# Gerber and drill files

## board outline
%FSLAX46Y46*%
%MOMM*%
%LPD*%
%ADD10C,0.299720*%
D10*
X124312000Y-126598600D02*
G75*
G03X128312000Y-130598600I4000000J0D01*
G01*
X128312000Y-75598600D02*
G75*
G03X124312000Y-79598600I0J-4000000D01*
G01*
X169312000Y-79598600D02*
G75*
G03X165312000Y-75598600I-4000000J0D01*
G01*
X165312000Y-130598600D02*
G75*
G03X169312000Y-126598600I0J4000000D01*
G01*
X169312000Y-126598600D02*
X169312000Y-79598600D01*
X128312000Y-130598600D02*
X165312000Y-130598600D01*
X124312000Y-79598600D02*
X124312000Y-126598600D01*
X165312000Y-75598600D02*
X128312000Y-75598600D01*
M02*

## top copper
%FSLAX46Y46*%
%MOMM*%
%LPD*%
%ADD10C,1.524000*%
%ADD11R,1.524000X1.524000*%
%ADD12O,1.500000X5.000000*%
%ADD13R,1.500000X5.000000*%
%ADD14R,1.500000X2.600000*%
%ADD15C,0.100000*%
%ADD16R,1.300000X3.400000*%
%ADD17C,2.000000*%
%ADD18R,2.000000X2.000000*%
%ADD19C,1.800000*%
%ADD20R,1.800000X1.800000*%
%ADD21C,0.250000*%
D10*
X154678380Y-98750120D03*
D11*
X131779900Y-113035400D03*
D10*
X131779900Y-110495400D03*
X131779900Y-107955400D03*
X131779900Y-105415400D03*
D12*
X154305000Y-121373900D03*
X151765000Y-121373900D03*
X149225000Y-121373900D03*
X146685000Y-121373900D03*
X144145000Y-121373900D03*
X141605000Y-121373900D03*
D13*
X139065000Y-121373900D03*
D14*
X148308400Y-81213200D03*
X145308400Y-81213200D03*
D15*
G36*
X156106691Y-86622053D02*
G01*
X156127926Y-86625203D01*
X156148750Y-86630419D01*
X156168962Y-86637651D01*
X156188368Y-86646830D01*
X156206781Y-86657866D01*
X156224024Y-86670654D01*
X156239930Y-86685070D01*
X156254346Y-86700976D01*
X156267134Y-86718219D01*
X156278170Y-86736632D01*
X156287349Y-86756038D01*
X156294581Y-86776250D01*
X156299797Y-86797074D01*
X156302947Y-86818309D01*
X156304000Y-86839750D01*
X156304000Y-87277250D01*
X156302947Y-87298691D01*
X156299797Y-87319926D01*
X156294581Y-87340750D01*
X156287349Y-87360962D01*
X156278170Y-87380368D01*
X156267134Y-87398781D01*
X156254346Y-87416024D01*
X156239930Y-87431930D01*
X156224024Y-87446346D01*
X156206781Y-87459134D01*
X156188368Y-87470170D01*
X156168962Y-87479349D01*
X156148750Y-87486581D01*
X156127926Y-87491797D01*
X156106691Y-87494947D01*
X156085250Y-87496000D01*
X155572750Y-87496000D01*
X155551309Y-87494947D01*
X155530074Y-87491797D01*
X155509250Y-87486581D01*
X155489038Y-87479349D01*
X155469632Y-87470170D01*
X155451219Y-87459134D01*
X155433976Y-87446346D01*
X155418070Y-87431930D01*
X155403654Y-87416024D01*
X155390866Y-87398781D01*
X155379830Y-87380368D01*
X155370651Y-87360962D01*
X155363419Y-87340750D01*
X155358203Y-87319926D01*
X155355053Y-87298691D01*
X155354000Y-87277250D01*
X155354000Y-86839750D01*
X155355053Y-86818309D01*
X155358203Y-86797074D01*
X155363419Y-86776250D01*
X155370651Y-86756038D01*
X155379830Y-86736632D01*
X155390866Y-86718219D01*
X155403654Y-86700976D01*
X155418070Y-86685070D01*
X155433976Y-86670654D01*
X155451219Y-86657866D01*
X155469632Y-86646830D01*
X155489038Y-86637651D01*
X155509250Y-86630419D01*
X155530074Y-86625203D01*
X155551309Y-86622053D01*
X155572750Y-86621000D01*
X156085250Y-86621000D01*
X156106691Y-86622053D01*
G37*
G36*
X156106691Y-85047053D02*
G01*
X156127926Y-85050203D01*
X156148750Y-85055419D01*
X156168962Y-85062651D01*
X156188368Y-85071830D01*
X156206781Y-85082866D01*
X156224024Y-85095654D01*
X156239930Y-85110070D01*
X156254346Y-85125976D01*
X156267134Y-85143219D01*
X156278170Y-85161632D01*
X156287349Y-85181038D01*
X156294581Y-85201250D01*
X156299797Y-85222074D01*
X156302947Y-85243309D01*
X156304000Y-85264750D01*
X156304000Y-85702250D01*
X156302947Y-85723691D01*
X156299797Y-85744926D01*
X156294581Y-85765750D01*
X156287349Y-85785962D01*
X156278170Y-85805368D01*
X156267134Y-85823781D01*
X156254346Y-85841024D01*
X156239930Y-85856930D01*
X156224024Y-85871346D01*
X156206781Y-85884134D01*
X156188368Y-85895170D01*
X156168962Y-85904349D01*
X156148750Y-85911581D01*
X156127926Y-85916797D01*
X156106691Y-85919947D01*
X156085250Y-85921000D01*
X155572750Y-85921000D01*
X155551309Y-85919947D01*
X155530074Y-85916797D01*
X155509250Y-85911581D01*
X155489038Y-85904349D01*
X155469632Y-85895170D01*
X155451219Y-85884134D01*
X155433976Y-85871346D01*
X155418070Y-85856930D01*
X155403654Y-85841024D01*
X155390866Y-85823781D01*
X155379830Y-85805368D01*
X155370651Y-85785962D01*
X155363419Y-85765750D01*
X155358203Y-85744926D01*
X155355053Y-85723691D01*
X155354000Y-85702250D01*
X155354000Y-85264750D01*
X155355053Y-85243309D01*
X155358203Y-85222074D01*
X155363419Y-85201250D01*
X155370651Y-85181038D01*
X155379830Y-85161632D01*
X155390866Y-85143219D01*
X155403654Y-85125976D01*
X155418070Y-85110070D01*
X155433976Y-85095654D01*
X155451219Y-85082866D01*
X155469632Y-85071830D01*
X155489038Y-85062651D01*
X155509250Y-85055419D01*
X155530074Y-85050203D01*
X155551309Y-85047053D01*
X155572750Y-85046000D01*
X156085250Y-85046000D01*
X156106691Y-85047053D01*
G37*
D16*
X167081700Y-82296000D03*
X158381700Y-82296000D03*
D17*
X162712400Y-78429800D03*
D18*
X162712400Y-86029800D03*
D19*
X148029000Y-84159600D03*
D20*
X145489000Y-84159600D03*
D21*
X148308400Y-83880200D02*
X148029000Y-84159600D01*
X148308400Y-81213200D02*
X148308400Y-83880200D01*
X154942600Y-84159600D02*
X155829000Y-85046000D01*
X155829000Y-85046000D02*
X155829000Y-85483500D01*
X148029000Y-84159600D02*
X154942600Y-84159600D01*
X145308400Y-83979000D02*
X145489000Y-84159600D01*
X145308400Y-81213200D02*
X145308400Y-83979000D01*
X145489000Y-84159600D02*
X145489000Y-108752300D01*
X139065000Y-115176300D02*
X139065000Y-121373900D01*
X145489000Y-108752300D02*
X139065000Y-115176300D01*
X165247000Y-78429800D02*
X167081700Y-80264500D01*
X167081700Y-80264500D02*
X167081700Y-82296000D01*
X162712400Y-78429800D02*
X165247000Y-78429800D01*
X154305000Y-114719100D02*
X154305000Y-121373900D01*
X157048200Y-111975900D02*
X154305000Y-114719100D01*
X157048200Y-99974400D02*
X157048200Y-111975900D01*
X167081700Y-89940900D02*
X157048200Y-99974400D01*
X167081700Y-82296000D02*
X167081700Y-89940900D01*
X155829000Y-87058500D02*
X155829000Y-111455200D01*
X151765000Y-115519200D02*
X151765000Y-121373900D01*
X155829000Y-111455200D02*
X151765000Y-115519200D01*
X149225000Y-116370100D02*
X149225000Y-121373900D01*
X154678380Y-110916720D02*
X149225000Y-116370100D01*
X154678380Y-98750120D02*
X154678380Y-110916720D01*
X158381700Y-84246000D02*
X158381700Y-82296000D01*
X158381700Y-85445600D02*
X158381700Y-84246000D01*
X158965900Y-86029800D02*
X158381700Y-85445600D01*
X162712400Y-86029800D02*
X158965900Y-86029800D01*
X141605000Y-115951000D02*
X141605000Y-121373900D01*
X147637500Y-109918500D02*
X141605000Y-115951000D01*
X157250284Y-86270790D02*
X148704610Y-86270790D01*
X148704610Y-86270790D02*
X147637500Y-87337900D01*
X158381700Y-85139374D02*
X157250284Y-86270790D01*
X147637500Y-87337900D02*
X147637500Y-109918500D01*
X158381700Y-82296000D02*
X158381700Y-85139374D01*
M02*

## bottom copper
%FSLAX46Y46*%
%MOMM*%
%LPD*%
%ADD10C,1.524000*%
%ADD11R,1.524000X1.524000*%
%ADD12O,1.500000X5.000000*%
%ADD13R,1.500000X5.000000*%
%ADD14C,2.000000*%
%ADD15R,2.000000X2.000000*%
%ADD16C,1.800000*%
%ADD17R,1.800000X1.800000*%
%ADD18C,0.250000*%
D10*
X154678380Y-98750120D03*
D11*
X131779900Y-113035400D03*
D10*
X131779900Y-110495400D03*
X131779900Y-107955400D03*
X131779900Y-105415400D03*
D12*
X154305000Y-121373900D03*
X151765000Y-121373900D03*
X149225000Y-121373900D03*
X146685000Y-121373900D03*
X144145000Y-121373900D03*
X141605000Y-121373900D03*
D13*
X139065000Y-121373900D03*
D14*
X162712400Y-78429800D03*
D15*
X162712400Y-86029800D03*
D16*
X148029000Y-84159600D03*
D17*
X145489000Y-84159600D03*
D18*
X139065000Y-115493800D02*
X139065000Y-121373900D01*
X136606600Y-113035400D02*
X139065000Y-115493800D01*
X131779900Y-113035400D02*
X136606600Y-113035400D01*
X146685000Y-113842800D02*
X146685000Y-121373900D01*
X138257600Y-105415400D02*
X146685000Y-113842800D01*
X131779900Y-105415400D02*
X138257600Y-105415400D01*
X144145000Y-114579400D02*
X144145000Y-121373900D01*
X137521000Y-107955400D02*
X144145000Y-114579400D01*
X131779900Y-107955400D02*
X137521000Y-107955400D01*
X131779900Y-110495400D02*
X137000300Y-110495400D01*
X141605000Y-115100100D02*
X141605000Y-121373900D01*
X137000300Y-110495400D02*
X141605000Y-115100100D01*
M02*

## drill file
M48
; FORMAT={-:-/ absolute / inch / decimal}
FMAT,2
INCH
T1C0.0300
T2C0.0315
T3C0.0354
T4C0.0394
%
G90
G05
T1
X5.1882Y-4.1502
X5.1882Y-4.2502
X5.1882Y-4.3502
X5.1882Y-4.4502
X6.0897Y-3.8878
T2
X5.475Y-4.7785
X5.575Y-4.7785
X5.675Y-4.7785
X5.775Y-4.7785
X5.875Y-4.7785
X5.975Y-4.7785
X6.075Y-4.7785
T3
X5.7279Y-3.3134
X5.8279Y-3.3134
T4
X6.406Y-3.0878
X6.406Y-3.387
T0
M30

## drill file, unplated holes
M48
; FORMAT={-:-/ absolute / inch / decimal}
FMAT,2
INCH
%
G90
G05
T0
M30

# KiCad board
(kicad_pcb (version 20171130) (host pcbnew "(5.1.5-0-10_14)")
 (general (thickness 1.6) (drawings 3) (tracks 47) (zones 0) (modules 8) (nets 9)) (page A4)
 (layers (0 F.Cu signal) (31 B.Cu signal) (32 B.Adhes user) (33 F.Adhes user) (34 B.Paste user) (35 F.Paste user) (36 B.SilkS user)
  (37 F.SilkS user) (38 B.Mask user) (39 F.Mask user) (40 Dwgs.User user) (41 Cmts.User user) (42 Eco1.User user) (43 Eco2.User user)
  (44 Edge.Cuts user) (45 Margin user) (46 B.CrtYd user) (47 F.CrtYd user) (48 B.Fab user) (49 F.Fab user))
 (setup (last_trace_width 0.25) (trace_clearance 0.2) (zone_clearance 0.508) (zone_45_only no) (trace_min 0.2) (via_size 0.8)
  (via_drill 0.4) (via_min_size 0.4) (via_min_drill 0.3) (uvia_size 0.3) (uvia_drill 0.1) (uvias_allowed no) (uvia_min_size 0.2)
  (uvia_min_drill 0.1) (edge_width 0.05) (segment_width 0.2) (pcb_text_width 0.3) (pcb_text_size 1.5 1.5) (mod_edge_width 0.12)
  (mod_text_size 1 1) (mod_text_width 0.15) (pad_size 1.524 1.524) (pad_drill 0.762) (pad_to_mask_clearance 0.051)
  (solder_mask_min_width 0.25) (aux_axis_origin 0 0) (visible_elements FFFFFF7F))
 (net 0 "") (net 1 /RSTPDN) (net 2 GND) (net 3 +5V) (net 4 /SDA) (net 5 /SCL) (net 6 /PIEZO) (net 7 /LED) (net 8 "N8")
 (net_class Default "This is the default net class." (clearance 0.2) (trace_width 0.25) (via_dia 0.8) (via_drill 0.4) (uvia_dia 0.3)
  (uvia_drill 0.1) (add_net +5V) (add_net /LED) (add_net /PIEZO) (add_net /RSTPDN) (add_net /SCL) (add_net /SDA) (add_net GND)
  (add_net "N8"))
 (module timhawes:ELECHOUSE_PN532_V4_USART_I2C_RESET (layer B.Cu) (at 151.5999 109.2454 90)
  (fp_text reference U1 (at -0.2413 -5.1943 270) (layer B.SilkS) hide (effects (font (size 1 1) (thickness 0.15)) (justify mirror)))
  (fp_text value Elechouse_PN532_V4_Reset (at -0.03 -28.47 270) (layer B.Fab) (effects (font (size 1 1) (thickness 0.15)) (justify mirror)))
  (pad 5 thru_hole circle (at 10.49528 3.07848 90) (size 1.524 1.524) (drill 0.762) (layers *.Cu *.Mask) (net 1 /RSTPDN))
  (pad 1 thru_hole rect (at -3.79 -19.82 90) (size 1.524 1.524) (drill 0.762) (layers *.Cu *.Mask) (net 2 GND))
  (pad 2 thru_hole circle (at -1.25 -19.82 90) (size 1.524 1.524) (drill 0.762) (layers *.Cu *.Mask) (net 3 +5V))
  (pad 3 thru_hole circle (at 1.29 -19.82 90) (size 1.524 1.524) (drill 0.762) (layers *.Cu *.Mask) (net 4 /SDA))
  (pad 4 thru_hole circle (at 3.83 -19.82 90) (size 1.524 1.524) (drill 0.762) (layers *.Cu *.Mask) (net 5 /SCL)))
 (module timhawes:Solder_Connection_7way (layer B.Cu) (at 146.685 121.3739)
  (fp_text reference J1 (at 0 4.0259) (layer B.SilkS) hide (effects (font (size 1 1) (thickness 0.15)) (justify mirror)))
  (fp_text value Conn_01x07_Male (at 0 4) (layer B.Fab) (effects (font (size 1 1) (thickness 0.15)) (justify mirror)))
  (pad 7 thru_hole oval (at 7.62 0) (size 1.5 5) (drill 0.8) (layers *.Cu *.Mask) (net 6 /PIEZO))
  (pad 6 thru_hole oval (at 5.08 0) (size 1.5 5) (drill 0.8) (layers *.Cu *.Mask) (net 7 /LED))
  (pad 5 thru_hole oval (at 2.54 0) (size 1.5 5) (drill 0.8) (layers *.Cu *.Mask) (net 1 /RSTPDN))
  (pad 4 thru_hole oval (at 0 0) (size 1.5 5) (drill 0.8) (layers *.Cu *.Mask) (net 5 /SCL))
  (pad 3 thru_hole oval (at -2.54 0) (size 1.5 5) (drill 0.8) (layers *.Cu *.Mask) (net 4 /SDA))
  (pad 2 thru_hole oval (at -5.08 0) (size 1.5 5) (drill 0.8) (layers *.Cu *.Mask) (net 3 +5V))
  (pad 1 thru_hole rect (at -7.62 0) (size 1.5 5) (drill 0.8) (layers *.Cu *.Mask) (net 2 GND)))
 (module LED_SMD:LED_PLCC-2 (layer F.Cu) (at 146.8084 81.2132)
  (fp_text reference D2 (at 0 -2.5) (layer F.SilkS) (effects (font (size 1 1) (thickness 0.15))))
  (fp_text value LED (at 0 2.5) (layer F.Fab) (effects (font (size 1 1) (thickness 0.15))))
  (pad 2 smd rect (at 1.5 0) (size 1.5 2.6) (layers F.Cu F.Paste F.Mask) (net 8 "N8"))
  (pad 1 smd rect (at -1.5 0) (size 1.5 2.6) (layers F.Cu F.Paste F.Mask) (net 2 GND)))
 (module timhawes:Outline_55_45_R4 (layer F.Cu) (at 146.812 103.0986 90)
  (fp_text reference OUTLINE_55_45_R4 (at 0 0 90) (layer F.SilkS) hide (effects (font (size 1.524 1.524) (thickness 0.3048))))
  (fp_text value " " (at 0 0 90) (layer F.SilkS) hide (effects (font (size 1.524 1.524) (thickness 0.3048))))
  (fp_arc (start -23.5 -18.5) (end -27.5 -18.5) (angle 90) (layer Edge.Cuts) (width 0.29972))
  (fp_arc (start 23.5 -18.5) (end 23.5 -22.5) (angle 90) (layer Edge.Cuts) (width 0.29972))
  (fp_arc (start 23.5 18.5) (end 27.5 18.5) (angle 90) (layer Edge.Cuts) (width 0.29972))
  (fp_arc (start -23.5 18.5) (end -23.5 22.5) (angle 90) (layer Edge.Cuts) (width 0.29972))
  (fp_line (start -23.5 22.5) (end 23.5 22.5) (layer Edge.Cuts) (width 0.29972))
  (fp_line (start -27.5 -18.5) (end -27.5 18.5) (layer Edge.Cuts) (width 0.29972))
  (fp_line (start 23.5 -22.5) (end -23.5 -22.5) (layer Edge.Cuts) (width 0.29972))
  (fp_line (start 27.5 18.5) (end 27.5 -18.5) (layer Edge.Cuts) (width 0.29972)))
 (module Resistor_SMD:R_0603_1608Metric (layer F.Cu) (at 155.829 86.271 270)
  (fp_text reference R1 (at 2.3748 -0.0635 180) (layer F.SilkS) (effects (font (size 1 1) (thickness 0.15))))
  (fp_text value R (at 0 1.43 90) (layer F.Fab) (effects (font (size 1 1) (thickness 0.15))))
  (pad 2 smd roundrect (at 0.7875 0 270) (size 0.875 0.95) (layers F.Cu F.Paste F.Mask) (roundrect_rratio 0.25) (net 7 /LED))
  (pad 1 smd roundrect (at -0.7875 0 270) (size 0.875 0.95) (layers F.Cu F.Paste F.Mask) (roundrect_rratio 0.25) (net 8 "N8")))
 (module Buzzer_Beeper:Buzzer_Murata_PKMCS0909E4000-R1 (layer F.Cu) (at 162.7317 82.296)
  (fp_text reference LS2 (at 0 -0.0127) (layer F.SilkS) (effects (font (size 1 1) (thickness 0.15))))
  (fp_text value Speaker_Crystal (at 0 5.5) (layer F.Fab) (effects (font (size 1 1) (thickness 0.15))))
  (pad 2 smd rect (at 4.35 0) (size 1.3 3.4) (layers F.Cu F.Paste F.Mask) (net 6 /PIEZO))
  (pad 1 smd rect (at -4.35 0) (size 1.3 3.4) (layers F.Cu F.Paste F.Mask) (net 3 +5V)))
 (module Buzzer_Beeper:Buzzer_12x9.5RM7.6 (layer B.Cu) (at 162.7124 86.0298 90)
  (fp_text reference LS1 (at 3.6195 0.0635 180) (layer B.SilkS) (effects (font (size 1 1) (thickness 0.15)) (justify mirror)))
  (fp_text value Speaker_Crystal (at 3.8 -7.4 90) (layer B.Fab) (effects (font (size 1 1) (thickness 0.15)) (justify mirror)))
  (pad 2 thru_hole circle (at 7.6 0 90) (size 2 2) (drill 1) (layers *.Cu *.Mask) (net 6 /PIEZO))
  (pad 1 thru_hole rect (at 0 0 90) (size 2 2) (drill 1) (layers *.Cu *.Mask) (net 3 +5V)))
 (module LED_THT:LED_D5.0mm (layer F.Cu) (at 145.489 84.1596)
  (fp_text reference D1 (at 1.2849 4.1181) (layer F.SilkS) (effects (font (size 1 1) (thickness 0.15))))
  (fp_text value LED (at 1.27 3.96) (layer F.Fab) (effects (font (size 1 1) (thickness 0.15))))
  (pad 2 thru_hole circle (at 2.54 0) (size 1.8 1.8) (drill 0.9) (layers *.Cu *.Mask) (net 8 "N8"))
  (pad 1 thru_hole rect (at 0 0) (size 1.8 1.8) (drill 0.9) (layers *.Cu *.Mask) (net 2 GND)))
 (segment (start 148.3084 83.8802) (end 148.029 84.1596) (width 0.25) (layer F.Cu) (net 8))
 (segment (start 148.3084 81.2132) (end 148.3084 83.8802) (width 0.25) (layer F.Cu) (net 8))
 (segment (start 154.9426 84.1596) (end 155.829 85.046) (width 0.25) (layer F.Cu) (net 8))
 (segment (start 155.829 85.046) (end 155.829 85.4835) (width 0.25) (layer F.Cu) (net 8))
 (segment (start 148.029 84.1596) (end 154.9426 84.1596) (width 0.25) (layer F.Cu) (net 8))
 (segment (start 145.3084 83.979) (end 145.489 84.1596) (width 0.25) (layer F.Cu) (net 2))
 (segment (start 145.3084 81.2132) (end 145.3084 83.979) (width 0.25) (layer F.Cu) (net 2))
 (segment (start 145.489 84.1596) (end 145.489 108.7523) (width 0.25) (layer F.Cu) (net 2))
 (segment (start 139.065 115.1763) (end 139.065 121.3739) (width 0.25) (layer F.Cu) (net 2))
 (segment (start 145.489 108.7523) (end 139.065 115.1763) (width 0.25) (layer F.Cu) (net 2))
 (segment (start 139.065 115.4938) (end 139.065 121.3739) (width 0.25) (layer B.Cu) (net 2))
 (segment (start 136.6066 113.0354) (end 139.065 115.4938) (width 0.25) (layer B.Cu) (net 2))
 (segment (start 131.7799 113.0354) (end 136.6066 113.0354) (width 0.25) (layer B.Cu) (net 2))
 (segment (start 165.247 78.4298) (end 167.0817 80.2645) (width 0.25) (layer F.Cu) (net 6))
 (segment (start 167.0817 80.2645) (end 167.0817 82.296) (width 0.25) (layer F.Cu) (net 6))
 (segment (start 162.7124 78.4298) (end 165.247 78.4298) (width 0.25) (layer F.Cu) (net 6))
 (segment (start 154.305 114.7191) (end 154.305 121.3739) (width 0.25) (layer F.Cu) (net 6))
 (segment (start 157.0482 111.9759) (end 154.305 114.7191) (width 0.25) (layer F.Cu) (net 6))
 (segment (start 157.0482 99.9744) (end 157.0482 111.9759) (width 0.25) (layer F.Cu) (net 6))
 (segment (start 167.0817 89.9409) (end 157.0482 99.9744) (width 0.25) (layer F.Cu) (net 6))
 (segment (start 167.0817 82.296) (end 167.0817 89.9409) (width 0.25) (layer F.Cu) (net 6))
 (segment (start 155.829 87.0585) (end 155.829 111.4552) (width 0.25) (layer F.Cu) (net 7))
 (segment (start 151.765 115.5192) (end 151.765 121.3739) (width 0.25) (layer F.Cu) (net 7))
 (segment (start 155.829 111.4552) (end 151.765 115.5192) (width 0.25) (layer F.Cu) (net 7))
 (segment (start 149.225 116.3701) (end 149.225 121.3739) (width 0.25) (layer F.Cu) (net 1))
 (segment (start 154.67838 110.91672) (end 149.225 116.3701) (width 0.25) (layer F.Cu) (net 1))
 (segment (start 154.67838 98.75012) (end 154.67838 110.91672) (width 0.25) (layer F.Cu) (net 1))
 (segment (start 146.685 113.8428) (end 146.685 121.3739) (width 0.25) (layer B.Cu) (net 5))
 (segment (start 138.2576 105.4154) (end 146.685 113.8428) (width 0.25) (layer B.Cu) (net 5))
 (segment (start 131.7799 105.4154) (end 138.2576 105.4154) (width 0.25) (layer B.Cu) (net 5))
 (segment (start 144.145 114.5794) (end 144.145 121.3739) (width 0.25) (layer B.Cu) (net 4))
 (segment (start 137.521 107.9554) (end 144.145 114.5794) (width 0.25) (layer B.Cu) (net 4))
 (segment (start 131.7799 107.9554) (end 137.521 107.9554) (width 0.25) (layer B.Cu) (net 4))
 (segment (start 158.3817 84.246) (end 158.3817 82.296) (width 0.25) (layer F.Cu) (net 3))
 (segment (start 158.3817 85.4456) (end 158.3817 84.246) (width 0.25) (layer F.Cu) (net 3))
 (segment (start 158.9659 86.0298) (end 158.3817 85.4456) (width 0.25) (layer F.Cu) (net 3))
 (segment (start 162.7124 86.0298) (end 158.9659 86.0298) (width 0.25) (layer F.Cu) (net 3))
 (segment (start 131.7799 110.4954) (end 137.0003 110.4954) (width 0.25) (layer B.Cu) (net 3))
 (segment (start 141.605 115.1001) (end 141.605 121.3739) (width 0.25) (layer B.Cu) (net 3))
 (segment (start 137.0003 110.4954) (end 141.605 115.1001) (width 0.25) (layer B.Cu) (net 3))
 (segment (start 141.605 115.951) (end 141.605 121.3739) (width 0.25) (layer F.Cu) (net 3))
 (segment (start 147.6375 109.9185) (end 141.605 115.951) (width 0.25) (layer F.Cu) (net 3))
 (segment (start 157.250284 86.27079) (end 148.70461 86.27079) (width 0.25) (layer F.Cu) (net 3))
 (segment (start 148.70461 86.27079) (end 147.6375 87.3379) (width 0.25) (layer F.Cu) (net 3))
 (segment (start 158.3817 85.139374) (end 157.250284 86.27079) (width 0.25) (layer F.Cu) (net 3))
 (segment (start 147.6375 87.3379) (end 147.6375 109.9185) (width 0.25) (layer F.Cu) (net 3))
 (segment (start 158.3817 82.296) (end 158.3817 85.139374) (width 0.25) (layer F.Cu) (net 3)))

